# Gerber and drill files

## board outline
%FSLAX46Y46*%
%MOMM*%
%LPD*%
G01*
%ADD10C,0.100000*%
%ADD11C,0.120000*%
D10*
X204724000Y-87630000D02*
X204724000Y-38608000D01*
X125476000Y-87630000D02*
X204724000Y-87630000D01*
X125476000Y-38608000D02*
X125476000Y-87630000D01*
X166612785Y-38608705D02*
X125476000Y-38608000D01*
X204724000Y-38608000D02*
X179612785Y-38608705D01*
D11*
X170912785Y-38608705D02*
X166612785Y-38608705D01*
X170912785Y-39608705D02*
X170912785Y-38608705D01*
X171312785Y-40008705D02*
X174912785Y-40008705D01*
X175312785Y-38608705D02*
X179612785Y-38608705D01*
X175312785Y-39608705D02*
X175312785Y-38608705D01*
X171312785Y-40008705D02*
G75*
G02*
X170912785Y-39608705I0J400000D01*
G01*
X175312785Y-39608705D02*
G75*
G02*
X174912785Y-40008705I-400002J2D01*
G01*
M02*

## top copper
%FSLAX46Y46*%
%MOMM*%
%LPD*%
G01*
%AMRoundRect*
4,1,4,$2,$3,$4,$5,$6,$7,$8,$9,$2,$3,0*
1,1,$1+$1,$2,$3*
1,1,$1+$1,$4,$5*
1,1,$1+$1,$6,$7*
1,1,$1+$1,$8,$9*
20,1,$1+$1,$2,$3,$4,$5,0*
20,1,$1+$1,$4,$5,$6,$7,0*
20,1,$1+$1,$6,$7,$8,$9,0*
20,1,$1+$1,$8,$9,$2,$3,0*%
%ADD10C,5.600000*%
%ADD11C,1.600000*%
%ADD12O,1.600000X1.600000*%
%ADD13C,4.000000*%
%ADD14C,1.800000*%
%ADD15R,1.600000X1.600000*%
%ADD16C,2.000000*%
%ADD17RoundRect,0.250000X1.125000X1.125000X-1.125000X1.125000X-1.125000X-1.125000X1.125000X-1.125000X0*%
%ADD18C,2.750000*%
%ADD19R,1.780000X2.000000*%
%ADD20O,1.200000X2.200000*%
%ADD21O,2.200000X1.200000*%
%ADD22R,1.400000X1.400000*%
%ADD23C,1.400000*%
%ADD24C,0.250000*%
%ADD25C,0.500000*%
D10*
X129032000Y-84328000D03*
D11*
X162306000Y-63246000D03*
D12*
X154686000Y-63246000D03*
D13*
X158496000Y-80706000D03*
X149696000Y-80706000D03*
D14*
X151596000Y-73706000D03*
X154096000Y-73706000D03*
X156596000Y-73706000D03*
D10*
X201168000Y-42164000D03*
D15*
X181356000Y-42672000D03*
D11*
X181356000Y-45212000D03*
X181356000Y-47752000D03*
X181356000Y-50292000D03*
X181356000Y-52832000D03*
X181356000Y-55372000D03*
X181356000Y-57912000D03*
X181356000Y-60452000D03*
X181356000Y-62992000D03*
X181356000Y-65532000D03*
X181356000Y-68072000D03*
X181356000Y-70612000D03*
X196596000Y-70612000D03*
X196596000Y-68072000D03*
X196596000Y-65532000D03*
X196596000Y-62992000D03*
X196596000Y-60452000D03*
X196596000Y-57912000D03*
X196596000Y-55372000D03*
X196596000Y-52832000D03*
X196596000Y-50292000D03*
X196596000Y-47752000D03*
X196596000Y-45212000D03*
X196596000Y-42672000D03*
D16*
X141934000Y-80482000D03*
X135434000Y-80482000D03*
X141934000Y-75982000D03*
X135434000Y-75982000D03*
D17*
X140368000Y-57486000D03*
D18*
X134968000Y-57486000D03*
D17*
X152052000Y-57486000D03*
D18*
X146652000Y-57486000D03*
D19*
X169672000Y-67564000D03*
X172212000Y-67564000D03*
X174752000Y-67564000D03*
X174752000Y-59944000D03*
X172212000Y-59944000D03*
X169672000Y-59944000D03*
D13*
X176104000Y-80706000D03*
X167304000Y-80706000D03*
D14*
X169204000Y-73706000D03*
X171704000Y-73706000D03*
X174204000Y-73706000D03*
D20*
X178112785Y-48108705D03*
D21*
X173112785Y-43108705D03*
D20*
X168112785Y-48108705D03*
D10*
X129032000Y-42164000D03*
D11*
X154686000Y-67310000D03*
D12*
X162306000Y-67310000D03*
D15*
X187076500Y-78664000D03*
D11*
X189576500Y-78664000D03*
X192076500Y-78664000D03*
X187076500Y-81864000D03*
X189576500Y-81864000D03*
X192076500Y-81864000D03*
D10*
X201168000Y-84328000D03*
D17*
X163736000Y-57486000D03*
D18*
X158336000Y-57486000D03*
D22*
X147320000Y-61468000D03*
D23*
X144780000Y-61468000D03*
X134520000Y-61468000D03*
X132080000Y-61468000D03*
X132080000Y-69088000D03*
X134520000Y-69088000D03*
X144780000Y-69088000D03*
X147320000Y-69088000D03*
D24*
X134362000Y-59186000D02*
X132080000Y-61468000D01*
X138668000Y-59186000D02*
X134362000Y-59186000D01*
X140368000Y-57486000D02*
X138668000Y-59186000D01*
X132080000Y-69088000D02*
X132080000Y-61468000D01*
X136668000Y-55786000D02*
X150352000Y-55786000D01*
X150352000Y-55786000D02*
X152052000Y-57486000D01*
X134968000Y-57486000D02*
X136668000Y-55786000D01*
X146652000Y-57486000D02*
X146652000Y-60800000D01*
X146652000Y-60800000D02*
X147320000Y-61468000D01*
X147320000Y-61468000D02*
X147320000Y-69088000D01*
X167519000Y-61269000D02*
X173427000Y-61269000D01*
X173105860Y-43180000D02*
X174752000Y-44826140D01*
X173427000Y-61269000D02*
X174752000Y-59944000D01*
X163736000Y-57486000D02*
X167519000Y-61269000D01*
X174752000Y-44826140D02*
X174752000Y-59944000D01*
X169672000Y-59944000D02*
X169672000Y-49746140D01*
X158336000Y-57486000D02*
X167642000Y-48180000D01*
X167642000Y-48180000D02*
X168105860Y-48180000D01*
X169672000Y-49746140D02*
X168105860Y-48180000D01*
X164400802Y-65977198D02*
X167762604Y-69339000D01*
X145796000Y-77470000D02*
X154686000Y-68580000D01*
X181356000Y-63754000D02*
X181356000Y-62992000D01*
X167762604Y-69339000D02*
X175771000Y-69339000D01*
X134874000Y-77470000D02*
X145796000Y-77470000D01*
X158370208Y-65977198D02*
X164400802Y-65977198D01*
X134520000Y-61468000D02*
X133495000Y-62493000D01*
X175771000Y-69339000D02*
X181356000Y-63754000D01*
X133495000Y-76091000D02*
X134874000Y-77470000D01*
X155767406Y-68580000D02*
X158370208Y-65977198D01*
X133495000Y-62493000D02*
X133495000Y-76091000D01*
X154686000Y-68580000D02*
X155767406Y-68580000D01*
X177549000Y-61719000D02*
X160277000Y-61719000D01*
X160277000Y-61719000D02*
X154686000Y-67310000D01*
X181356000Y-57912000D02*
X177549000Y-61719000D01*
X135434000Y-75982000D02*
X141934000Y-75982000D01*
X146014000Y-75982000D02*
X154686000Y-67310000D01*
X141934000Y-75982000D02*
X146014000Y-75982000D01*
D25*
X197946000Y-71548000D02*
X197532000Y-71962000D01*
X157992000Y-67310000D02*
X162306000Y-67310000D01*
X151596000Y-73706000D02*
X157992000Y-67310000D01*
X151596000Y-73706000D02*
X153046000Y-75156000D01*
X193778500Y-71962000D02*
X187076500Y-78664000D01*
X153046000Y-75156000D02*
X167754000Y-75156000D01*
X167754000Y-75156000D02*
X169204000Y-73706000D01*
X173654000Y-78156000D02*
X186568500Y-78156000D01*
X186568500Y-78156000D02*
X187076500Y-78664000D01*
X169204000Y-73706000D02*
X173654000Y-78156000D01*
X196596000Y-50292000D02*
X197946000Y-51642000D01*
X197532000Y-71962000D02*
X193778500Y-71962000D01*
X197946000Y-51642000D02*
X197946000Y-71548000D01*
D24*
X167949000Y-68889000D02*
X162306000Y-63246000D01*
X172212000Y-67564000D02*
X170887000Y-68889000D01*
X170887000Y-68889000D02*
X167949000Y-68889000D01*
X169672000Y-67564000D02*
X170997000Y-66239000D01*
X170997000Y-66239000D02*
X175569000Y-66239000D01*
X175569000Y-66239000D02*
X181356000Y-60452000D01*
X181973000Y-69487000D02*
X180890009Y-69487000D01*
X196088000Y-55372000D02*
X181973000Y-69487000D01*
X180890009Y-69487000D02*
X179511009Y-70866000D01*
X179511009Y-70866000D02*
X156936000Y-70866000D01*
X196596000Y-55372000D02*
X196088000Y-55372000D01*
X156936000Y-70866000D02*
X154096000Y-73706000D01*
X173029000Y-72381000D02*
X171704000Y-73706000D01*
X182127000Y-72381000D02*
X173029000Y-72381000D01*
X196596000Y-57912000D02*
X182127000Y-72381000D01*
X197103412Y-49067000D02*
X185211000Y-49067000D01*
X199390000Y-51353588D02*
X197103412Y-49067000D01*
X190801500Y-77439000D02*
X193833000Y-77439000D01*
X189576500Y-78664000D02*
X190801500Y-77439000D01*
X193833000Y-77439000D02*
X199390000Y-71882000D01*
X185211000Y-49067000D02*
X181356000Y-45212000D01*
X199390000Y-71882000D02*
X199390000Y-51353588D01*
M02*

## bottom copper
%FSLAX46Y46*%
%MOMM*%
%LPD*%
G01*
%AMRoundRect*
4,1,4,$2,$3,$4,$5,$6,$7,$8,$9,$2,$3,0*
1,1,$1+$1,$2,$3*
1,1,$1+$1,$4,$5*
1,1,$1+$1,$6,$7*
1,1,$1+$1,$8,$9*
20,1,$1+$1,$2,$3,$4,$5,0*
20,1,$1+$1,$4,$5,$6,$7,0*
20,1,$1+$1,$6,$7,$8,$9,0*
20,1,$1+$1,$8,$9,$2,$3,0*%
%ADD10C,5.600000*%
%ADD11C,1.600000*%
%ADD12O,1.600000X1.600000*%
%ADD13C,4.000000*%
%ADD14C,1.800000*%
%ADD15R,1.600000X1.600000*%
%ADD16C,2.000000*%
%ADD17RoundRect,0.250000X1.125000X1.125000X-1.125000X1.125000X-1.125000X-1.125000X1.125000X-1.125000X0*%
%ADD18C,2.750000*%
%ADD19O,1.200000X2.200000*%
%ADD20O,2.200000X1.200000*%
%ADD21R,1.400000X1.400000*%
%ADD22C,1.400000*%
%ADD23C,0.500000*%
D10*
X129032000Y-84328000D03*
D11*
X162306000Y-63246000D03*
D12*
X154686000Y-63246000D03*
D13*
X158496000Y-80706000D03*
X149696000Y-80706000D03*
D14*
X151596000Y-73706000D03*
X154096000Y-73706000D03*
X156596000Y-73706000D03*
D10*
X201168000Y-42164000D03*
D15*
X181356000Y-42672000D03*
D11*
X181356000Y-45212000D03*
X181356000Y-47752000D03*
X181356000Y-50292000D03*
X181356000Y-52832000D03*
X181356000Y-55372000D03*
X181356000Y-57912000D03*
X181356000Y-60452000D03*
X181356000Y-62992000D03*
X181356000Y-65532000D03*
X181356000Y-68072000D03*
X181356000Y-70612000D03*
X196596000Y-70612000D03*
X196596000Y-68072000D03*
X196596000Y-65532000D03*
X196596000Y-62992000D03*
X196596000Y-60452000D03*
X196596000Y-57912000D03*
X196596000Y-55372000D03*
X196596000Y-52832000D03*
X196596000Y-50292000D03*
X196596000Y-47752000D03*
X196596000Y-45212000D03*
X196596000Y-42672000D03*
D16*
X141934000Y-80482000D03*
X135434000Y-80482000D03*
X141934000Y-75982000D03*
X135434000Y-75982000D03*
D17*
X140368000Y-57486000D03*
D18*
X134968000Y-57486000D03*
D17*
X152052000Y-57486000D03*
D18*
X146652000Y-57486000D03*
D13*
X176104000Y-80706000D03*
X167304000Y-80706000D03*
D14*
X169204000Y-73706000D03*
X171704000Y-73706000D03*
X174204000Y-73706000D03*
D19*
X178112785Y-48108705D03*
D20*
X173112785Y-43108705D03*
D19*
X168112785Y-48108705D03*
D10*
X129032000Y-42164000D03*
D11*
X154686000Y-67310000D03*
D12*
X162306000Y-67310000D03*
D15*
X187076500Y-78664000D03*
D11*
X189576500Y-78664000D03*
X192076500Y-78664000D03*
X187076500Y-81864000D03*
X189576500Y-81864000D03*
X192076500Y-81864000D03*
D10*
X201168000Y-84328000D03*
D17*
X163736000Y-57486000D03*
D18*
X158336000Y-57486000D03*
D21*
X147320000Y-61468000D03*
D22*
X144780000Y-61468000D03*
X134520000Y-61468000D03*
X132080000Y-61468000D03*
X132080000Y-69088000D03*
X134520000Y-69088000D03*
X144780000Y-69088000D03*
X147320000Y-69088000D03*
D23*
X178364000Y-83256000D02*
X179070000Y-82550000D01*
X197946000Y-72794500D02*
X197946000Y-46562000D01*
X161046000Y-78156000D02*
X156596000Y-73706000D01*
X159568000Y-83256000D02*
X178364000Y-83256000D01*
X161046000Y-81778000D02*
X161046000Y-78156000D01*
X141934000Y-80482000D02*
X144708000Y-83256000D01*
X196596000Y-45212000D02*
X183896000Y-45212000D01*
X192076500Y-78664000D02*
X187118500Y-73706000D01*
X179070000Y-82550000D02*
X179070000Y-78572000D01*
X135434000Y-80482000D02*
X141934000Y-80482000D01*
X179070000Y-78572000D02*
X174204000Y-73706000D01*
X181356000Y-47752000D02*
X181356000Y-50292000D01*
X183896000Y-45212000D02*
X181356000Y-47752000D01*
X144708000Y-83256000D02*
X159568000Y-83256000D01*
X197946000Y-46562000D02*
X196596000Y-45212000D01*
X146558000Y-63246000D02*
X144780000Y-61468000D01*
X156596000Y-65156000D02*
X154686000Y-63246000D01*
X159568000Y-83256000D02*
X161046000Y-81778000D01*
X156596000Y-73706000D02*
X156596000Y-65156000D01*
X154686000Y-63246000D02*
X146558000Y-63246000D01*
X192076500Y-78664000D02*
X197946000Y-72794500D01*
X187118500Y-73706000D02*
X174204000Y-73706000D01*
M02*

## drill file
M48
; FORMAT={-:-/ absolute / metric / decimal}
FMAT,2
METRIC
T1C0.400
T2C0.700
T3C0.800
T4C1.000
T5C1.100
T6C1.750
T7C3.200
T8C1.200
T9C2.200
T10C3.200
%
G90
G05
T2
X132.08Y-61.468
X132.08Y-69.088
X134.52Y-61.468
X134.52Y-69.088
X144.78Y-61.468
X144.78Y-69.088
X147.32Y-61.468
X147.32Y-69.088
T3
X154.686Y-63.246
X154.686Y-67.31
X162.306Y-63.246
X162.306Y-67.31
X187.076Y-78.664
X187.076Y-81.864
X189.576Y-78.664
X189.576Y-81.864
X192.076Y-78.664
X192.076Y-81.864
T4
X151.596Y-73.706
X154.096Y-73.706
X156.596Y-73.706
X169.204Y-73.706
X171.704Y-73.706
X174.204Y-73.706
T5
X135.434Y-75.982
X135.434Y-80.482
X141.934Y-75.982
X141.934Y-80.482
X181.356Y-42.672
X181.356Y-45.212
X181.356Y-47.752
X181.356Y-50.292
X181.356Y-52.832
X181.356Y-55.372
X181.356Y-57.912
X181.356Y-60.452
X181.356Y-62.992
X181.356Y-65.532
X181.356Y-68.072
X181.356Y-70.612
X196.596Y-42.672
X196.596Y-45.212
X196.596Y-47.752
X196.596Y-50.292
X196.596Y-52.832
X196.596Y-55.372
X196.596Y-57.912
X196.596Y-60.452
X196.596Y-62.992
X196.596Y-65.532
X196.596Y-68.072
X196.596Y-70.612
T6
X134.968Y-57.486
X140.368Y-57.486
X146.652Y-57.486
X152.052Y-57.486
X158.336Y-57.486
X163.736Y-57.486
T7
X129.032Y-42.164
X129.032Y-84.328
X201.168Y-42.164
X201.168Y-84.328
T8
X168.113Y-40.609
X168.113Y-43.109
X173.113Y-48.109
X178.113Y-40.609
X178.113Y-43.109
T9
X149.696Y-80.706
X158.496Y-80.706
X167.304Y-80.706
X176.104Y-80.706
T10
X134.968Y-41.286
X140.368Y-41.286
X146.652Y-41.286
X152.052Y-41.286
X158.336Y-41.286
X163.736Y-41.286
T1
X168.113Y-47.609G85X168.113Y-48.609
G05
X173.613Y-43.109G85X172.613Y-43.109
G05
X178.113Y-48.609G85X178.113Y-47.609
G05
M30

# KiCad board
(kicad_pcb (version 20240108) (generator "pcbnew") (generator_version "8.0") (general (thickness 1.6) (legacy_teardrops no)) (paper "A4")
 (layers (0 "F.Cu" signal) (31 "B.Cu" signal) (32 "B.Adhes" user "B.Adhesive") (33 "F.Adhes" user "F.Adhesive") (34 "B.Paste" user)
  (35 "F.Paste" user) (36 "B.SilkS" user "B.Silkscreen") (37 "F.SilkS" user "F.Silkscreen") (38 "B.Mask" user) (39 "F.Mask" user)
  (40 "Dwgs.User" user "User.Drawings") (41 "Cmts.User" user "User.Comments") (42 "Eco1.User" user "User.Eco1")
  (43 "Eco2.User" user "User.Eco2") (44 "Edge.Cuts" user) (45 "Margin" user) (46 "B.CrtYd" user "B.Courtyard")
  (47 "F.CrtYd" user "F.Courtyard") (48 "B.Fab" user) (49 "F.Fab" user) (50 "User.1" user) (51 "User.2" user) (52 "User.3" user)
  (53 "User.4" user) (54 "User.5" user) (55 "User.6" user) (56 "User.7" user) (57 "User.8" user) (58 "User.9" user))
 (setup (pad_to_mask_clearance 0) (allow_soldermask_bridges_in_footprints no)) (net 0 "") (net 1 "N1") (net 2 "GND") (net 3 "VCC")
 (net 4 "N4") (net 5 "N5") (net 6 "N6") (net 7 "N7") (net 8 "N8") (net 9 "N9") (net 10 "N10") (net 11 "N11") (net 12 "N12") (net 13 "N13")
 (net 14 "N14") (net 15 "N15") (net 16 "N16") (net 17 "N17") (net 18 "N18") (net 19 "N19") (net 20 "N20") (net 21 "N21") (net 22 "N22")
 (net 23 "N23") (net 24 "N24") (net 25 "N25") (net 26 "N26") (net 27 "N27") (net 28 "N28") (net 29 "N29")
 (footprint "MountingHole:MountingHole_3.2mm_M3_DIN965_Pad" (layer "F.Cu") (at 129.032 84.328)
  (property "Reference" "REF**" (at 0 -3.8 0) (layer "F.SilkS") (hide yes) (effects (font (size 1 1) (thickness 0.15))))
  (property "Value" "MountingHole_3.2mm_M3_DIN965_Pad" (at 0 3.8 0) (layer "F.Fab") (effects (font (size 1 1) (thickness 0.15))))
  (pad "1" thru_hole circle (at 0 0) (size 5.6 5.6) (drill 3.2) (layers "*.Cu" "*.Mask") (remove_unused_layers no)))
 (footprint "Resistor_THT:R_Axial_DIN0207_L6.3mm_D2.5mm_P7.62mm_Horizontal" (layer "F.Cu") (at 162.306 63.246 180)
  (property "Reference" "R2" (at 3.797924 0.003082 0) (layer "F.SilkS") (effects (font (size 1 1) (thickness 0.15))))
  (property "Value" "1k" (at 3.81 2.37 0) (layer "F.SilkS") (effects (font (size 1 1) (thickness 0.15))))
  (pad "1" thru_hole circle (at 0 0 180) (size 1.6 1.6) (drill 0.8) (layers "*.Cu" "*.Mask") (remove_unused_layers no) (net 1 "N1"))
  (pad "2" thru_hole oval (at 7.62 0 180) (size 1.6 1.6) (drill 0.8) (layers "*.Cu" "*.Mask") (remove_unused_layers no) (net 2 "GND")))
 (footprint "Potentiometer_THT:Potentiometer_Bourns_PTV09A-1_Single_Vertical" (layer "F.Cu") (at 151.596 73.706 -90)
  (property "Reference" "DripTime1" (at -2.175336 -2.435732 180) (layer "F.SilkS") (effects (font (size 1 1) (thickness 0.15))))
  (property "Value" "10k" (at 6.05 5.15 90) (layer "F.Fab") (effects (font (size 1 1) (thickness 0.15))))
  (pad "" np_thru_hole circle (at 7 -6.9 270) (size 4 4) (drill 2.2) (layers "F&B.Cu" "*.Mask"))
  (pad "" np_thru_hole circle (at 7 1.9 270) (size 4 4) (drill 2.2) (layers "F&B.Cu" "*.Mask"))
  (pad "1" thru_hole circle (at 0 0 270) (size 1.8 1.8) (drill 1) (layers "*.Cu" "*.Mask") (remove_unused_layers no) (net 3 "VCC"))
  (pad "2" thru_hole circle (at 0 -2.5 270) (size 1.8 1.8) (drill 1) (layers "*.Cu" "*.Mask") (remove_unused_layers no) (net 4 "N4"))
  (pad "3" thru_hole circle (at 0 -5 270) (size 1.8 1.8) (drill 1) (layers "*.Cu" "*.Mask") (remove_unused_layers no) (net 2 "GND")))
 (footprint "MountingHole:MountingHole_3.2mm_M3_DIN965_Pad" (layer "F.Cu") (at 201.168 42.164)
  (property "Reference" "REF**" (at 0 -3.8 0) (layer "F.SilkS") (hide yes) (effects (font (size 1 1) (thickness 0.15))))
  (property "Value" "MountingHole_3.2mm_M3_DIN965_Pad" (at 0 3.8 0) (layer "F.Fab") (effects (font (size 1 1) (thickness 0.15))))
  (pad "1" thru_hole circle (at 0 0) (size 5.6 5.6) (drill 3.2) (layers "*.Cu" "*.Mask") (remove_unused_layers no)))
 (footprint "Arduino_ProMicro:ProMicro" (layer "F.Cu") (at 188.976 56.642 -90)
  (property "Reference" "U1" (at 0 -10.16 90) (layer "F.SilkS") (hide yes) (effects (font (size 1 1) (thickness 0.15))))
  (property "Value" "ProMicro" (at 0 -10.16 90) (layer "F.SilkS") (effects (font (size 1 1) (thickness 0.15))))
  (pad "1" thru_hole rect (at -13.97 7.62 270) (size 1.6 1.6) (drill 1.1) (layers "*.Cu" "*.Mask" "F.SilkS") (remove_unused_layers no)
   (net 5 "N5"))
  (pad "2" thru_hole circle (at -11.43 7.62 270) (size 1.6 1.6) (drill 1.1) (layers "*.Cu" "*.Mask" "F.SilkS") (remove_unused_layers no)
   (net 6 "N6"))
  (pad "3" thru_hole circle (at -8.89 7.62 270) (size 1.6 1.6) (drill 1.1) (layers "*.Cu" "*.Mask" "F.SilkS") (remove_unused_layers no)
   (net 2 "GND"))
  (pad "4" thru_hole circle (at -6.35 7.62 270) (size 1.6 1.6) (drill 1.1) (layers "*.Cu" "*.Mask" "F.SilkS") (remove_unused_layers no)
   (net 2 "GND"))
  (pad "5" thru_hole circle (at -3.81 7.62 270) (size 1.6 1.6) (drill 1.1) (layers "*.Cu" "*.Mask" "F.SilkS") (remove_unused_layers no)
   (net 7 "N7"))
  (pad "6" thru_hole circle (at -1.27 7.62 270) (size 1.6 1.6) (drill 1.1) (layers "*.Cu" "*.Mask" "F.SilkS") (remove_unused_layers no)
   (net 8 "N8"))
  (pad "7" thru_hole circle (at 1.27 7.62 270) (size 1.6 1.6) (drill 1.1) (layers "*.Cu" "*.Mask" "F.SilkS") (remove_unused_layers no)
   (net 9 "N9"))
  (pad "8" thru_hole circle (at 3.81 7.62 270) (size 1.6 1.6) (drill 1.1) (layers "*.Cu" "*.Mask" "F.SilkS") (remove_unused_layers no)
   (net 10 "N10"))
  (pad "9" thru_hole circle (at 6.35 7.62 270) (size 1.6 1.6) (drill 1.1) (layers "*.Cu" "*.Mask" "F.SilkS") (remove_unused_layers no)
   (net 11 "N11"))
  (pad "10" thru_hole circle (at 8.89 7.62 270) (size 1.6 1.6) (drill 1.1) (layers "*.Cu" "*.Mask" "F.SilkS") (remove_unused_layers no)
   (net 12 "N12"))
  (pad "11" thru_hole circle (at 11.43 7.62 270) (size 1.6 1.6) (drill 1.1) (layers "*.Cu" "*.Mask" "F.SilkS") (remove_unused_layers no)
   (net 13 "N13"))
  (pad "12" thru_hole circle (at 13.97 7.62 270) (size 1.6 1.6) (drill 1.1) (layers "*.Cu" "*.Mask" "F.SilkS") (remove_unused_layers no)
   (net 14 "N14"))
  (pad "13" thru_hole circle (at 13.97 -7.62 270) (size 1.6 1.6) (drill 1.1) (layers "*.Cu" "*.Mask" "F.SilkS") (remove_unused_layers no)
   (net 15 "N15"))
  (pad "14" thru_hole circle (at 11.43 -7.62 270) (size 1.6 1.6) (drill 1.1) (layers "*.Cu" "*.Mask" "F.SilkS") (remove_unused_layers no)
   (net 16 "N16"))
  (pad "15" thru_hole circle (at 8.89 -7.62 270) (size 1.6 1.6) (drill 1.1) (layers "*.Cu" "*.Mask" "F.SilkS") (remove_unused_layers no)
   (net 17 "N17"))
  (pad "16" thru_hole circle (at 6.35 -7.62 270) (size 1.6 1.6) (drill 1.1) (layers "*.Cu" "*.Mask" "F.SilkS") (remove_unused_layers no)
   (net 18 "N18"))
  (pad "17" thru_hole circle (at 3.81 -7.62 270) (size 1.6 1.6) (drill 1.1) (layers "*.Cu" "*.Mask" "F.SilkS") (remove_unused_layers no)
   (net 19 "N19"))
  (pad "18" thru_hole circle (at 1.27 -7.62 270) (size 1.6 1.6) (drill 1.1) (layers "*.Cu" "*.Mask" "F.SilkS") (remove_unused_layers no)
   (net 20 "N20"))
  (pad "19" thru_hole circle (at -1.27 -7.62 270) (size 1.6 1.6) (drill 1.1) (layers "*.Cu" "*.Mask" "F.SilkS") (remove_unused_layers no)
   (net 4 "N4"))
  (pad "20" thru_hole circle (at -3.81 -7.62 270) (size 1.6 1.6) (drill 1.1) (layers "*.Cu" "*.Mask" "F.SilkS") (remove_unused_layers no)
   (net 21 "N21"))
  (pad "21" thru_hole circle (at -6.35 -7.62 270) (size 1.6 1.6) (drill 1.1) (layers "*.Cu" "*.Mask" "F.SilkS") (remove_unused_layers no)
   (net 3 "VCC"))
  (pad "22" thru_hole circle (at -8.89 -7.62 270) (size 1.6 1.6) (drill 1.1) (layers "*.Cu" "*.Mask" "F.SilkS") (remove_unused_layers no)
   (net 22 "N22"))
  (pad "23" thru_hole circle (at -11.43 -7.62 270) (size 1.6 1.6) (drill 1.1) (layers "*.Cu" "*.Mask" "F.SilkS") (remove_unused_layers no)
   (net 2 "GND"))
  (pad "24" thru_hole circle (at -13.97 -7.62 270) (size 1.6 1.6) (drill 1.1) (layers "*.Cu" "*.Mask" "F.SilkS") (remove_unused_layers no)
   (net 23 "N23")))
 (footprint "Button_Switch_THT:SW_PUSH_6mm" (layer "F.Cu") (at 141.934 80.482 180)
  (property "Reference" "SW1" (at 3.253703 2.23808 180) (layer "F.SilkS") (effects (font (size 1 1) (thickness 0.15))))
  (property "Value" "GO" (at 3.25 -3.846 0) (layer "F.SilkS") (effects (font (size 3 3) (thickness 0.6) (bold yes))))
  (pad "1" thru_hole circle (at 0 0 270) (size 2 2) (drill 1.1) (layers "*.Cu" "*.Mask") (remove_unused_layers no) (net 2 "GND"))
  (pad "1" thru_hole circle (at 6.5 0 270) (size 2 2) (drill 1.1) (layers "*.Cu" "*.Mask") (remove_unused_layers no) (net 2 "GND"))
  (pad "2" thru_hole circle (at 0 4.5 270) (size 2 2) (drill 1.1) (layers "*.Cu" "*.Mask") (remove_unused_layers no) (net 9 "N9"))
  (pad "2" thru_hole circle (at 6.5 4.5 270) (size 2 2) (drill 1.1) (layers "*.Cu" "*.Mask") (remove_unused_layers no) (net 9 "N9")))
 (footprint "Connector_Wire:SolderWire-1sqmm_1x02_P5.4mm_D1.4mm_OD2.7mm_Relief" (layer "F.Cu") (at 140.368 57.486 180)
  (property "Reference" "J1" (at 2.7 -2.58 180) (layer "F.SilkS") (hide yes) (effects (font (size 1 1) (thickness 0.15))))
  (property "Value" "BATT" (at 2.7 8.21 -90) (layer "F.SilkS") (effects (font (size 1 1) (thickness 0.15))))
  (pad "" np_thru_hole circle (at 0 16.2 180) (size 3.2 3.2) (drill 3.2) (layers "*.Cu" "*.Mask"))
  (pad "" np_thru_hole circle (at 5.4 16.2 180) (size 3.2 3.2) (drill 3.2) (layers "*.Cu" "*.Mask"))
  (pad "1" thru_hole roundrect (at 0 0 180) (size 2.75 2.75) (drill 1.75) (layers "*.Cu" "*.Mask") (remove_unused_layers no)
   (roundrect_rratio 0.090909) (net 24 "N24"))
  (pad "2" thru_hole circle (at 5.4 0 180) (size 2.75 2.75) (drill 1.75) (layers "*.Cu" "*.Mask") (remove_unused_layers no) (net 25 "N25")))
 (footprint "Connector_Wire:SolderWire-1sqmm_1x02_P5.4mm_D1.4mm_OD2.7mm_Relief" (layer "F.Cu") (at 152.052 57.486 180)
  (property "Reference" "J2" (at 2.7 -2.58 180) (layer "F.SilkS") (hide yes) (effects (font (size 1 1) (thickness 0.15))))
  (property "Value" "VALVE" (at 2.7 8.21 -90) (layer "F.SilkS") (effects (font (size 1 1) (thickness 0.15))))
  (pad "" np_thru_hole circle (at 0 16.2 180) (size 3.2 3.2) (drill 3.2) (layers "*.Cu" "*.Mask"))
  (pad "" np_thru_hole circle (at 5.4 16.2 180) (size 3.2 3.2) (drill 3.2) (layers "*.Cu" "*.Mask"))
  (pad "1" thru_hole roundrect (at 0 0 180) (size 2.75 2.75) (drill 1.75) (layers "*.Cu" "*.Mask") (remove_unused_layers no)
   (roundrect_rratio 0.090909) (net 25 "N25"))
  (pad "2" thru_hole circle (at 5.4 0 180) (size 2.75 2.75) (drill 1.75) (layers "*.Cu" "*.Mask") (remove_unused_layers no) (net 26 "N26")))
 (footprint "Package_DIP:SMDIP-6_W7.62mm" (layer "F.Cu") (at 172.212 63.754 90)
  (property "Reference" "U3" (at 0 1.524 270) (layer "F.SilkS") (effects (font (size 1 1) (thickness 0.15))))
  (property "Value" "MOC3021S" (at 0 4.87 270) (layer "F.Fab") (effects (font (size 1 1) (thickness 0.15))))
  (pad "1" smd rect (at -3.81 -2.54 90) (size 2 1.78) (layers "F.Cu" "F.Paste" "F.Mask") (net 10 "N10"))
  (pad "2" smd rect (at -3.81 0 90) (size 2 1.78) (layers "F.Cu" "F.Paste" "F.Mask") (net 1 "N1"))
  (pad "3" smd rect (at -3.81 2.54 90) (size 2 1.78) (layers "F.Cu" "F.Paste" "F.Mask") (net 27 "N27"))
  (pad "4" smd rect (at 3.81 2.54 90) (size 2 1.78) (layers "F.Cu" "F.Paste" "F.Mask") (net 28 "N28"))
  (pad "5" smd rect (at 3.81 0 90) (size 2 1.78) (layers "F.Cu" "F.Paste" "F.Mask"))
  (pad "6" smd rect (at 3.81 -2.54 90) (size 2 1.78) (layers "F.Cu" "F.Paste" "F.Mask") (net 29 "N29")))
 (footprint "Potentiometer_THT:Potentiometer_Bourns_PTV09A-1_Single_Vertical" (layer "F.Cu") (at 169.204 73.706 -90)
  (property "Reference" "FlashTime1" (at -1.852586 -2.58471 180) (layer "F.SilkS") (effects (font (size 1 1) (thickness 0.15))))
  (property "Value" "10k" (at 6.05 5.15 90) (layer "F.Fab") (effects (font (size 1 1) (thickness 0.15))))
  (pad "" np_thru_hole circle (at 7 -6.9 270) (size 4 4) (drill 2.2) (layers "F&B.Cu" "*.Mask"))
  (pad "" np_thru_hole circle (at 7 1.9 270) (size 4 4) (drill 2.2) (layers "F&B.Cu" "*.Mask"))
  (pad "1" thru_hole circle (at 0 0 270) (size 1.8 1.8) (drill 1) (layers "*.Cu" "*.Mask") (remove_unused_layers no) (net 3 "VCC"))
  (pad "2" thru_hole circle (at 0 -2.5 270) (size 1.8 1.8) (drill 1) (layers "*.Cu" "*.Mask") (remove_unused_layers no) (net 20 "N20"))
  (pad "3" thru_hole circle (at 0 -5 270) (size 1.8 1.8) (drill 1) (layers "*.Cu" "*.Mask") (remove_unused_layers no) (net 2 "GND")))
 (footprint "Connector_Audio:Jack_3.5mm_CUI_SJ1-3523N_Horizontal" (layer "F.Cu") (at 173.112785 43.108705 180)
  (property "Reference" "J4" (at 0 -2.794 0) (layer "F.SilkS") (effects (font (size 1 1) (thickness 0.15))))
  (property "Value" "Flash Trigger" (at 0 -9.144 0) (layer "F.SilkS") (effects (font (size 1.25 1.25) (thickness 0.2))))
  (fp_line (start 2.2 4.5) (end 6.5 4.5) (stroke (width 0.12) (type solid)) (layer "Edge.Cuts"))
  (fp_line (start 2.2 3.5) (end 2.2 4.5) (stroke (width 0.12) (type solid)) (layer "Edge.Cuts"))
  (fp_line (start 1.8 3.1) (end -1.8 3.1) (stroke (width 0.12) (type solid)) (layer "Edge.Cuts"))
  (fp_line (start -2.2 4.5) (end -6.5 4.5) (stroke (width 0.12) (type solid)) (layer "Edge.Cuts"))
  (fp_line (start -2.2 3.5) (end -2.2 4.5) (stroke (width 0.12) (type solid)) (layer "Edge.Cuts"))
  (fp_arc (start 1.8 3.1) (mid 2.082843 3.217157) (end 2.2 3.5) (stroke (width 0.12) (type solid)) (layer "Edge.Cuts"))
  (fp_arc (start -2.2 3.5) (mid -2.082842 3.217158) (end -1.8 3.1) (stroke (width 0.12) (type solid)) (layer "Edge.Cuts"))
  (pad "" np_thru_hole circle (at -5 0 180) (size 1.2 1.2) (drill 1.2) (layers "*.Cu"))
  (pad "" np_thru_hole circle (at -5 2.5 180) (size 1.2 1.2) (drill 1.2) (layers "*.Cu"))
  (pad "" np_thru_hole circle (at 0 -5 180) (size 1.2 1.2) (drill 1.2) (layers "*.Cu"))
  (pad "" np_thru_hole circle (at 5 0 180) (size 1.2 1.2) (drill 1.2) (layers "*.Cu"))
  (pad "" np_thru_hole circle (at 5 2.5 180) (size 1.2 1.2) (drill 1.2) (layers "*.Cu"))
  (pad "R" thru_hole oval (at -5 -5 180) (size 1.2 2.2) (drill oval 0.4 1.4) (layers "*.Cu" "*.Mask") (remove_unused_layers no))
  (pad "S" thru_hole oval (at 0 0 180) (size 2.2 1.2) (drill oval 1.4 0.4) (layers "*.Cu" "*.Mask") (remove_unused_layers no) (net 28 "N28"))
  (pad "T" thru_hole oval (at 5 -5) (size 1.2 2.2) (drill oval 0.4 1.4) (layers "*.Cu" "*.Mask") (remove_unused_layers no) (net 29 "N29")))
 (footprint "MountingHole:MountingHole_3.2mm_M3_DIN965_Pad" (layer "F.Cu") (at 129.032 42.164)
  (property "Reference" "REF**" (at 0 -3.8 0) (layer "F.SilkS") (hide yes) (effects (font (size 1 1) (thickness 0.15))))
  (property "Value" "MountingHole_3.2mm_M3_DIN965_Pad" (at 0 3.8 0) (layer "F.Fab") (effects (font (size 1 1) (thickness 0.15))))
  (pad "1" thru_hole circle (at 0 0) (size 5.6 5.6) (drill 3.2) (layers "*.Cu" "*.Mask") (remove_unused_layers no)))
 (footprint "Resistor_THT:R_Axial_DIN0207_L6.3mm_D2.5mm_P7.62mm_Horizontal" (layer "F.Cu") (at 154.686 67.31)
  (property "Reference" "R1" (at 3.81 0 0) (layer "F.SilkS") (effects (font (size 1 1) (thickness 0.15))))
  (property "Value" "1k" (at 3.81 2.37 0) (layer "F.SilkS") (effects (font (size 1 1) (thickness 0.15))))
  (pad "1" thru_hole circle (at 0 0) (size 1.6 1.6) (drill 0.8) (layers "*.Cu" "*.Mask") (remove_unused_layers no) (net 9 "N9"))
  (pad "2" thru_hole oval (at 7.62 0) (size 1.6 1.6) (drill 0.8) (layers "*.Cu" "*.Mask") (remove_unused_layers no) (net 3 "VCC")))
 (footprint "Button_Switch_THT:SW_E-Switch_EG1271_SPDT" (layer "F.Cu") (at 187.0765 78.664)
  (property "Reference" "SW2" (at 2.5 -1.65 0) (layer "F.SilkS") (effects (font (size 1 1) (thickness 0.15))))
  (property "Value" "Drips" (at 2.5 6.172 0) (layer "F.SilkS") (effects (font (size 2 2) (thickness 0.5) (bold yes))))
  (pad "1" thru_hole rect (at 0 0) (size 1.6 1.6) (drill 0.8) (layers "*.Cu" "*.Mask") (remove_unused_layers no) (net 3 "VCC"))
  (pad "2" thru_hole circle (at 2.5 0) (size 1.6 1.6) (drill 0.8) (layers "*.Cu" "*.Mask") (remove_unused_layers no) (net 6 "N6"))
  (pad "3" thru_hole circle (at 5 0) (size 1.6 1.6) (drill 0.8) (layers "*.Cu" "*.Mask") (remove_unused_layers no) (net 2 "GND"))
  (pad "4" thru_hole circle (at 0 3.2) (size 1.6 1.6) (drill 0.8) (layers "*.Cu" "*.Mask") (remove_unused_layers no))
  (pad "5" thru_hole circle (at 2.5 3.2) (size 1.6 1.6) (drill 0.8) (layers "*.Cu" "*.Mask") (remove_unused_layers no))
  (pad "6" thru_hole circle (at 5 3.2) (size 1.6 1.6) (drill 0.8) (layers "*.Cu" "*.Mask") (remove_unused_layers no)))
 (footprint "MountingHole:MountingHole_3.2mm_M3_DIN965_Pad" (layer "F.Cu") (at 201.168 84.328)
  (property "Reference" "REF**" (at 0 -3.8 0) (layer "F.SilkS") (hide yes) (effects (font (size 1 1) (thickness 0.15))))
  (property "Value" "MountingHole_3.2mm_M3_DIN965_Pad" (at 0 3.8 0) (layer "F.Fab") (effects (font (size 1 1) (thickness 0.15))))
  (pad "1" thru_hole circle (at 0 0) (size 5.6 5.6) (drill 3.2) (layers "*.Cu" "*.Mask") (remove_unused_layers no)))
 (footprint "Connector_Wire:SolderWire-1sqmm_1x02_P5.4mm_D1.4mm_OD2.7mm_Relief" (layer "F.Cu") (at 163.736 57.486 180)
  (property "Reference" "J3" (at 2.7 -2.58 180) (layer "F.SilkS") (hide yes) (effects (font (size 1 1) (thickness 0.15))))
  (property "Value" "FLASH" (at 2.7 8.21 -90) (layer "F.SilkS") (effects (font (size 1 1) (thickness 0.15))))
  (pad "" np_thru_hole circle (at 0 16.2 180) (size 3.2 3.2) (drill 3.2) (layers "*.Cu" "*.Mask"))
  (pad "" np_thru_hole circle (at 5.4 16.2 180) (size 3.2 3.2) (drill 3.2) (layers "*.Cu" "*.Mask"))
  (pad "1" thru_hole roundrect (at 0 0 180) (size 2.75 2.75) (drill 1.75) (layers "*.Cu" "*.Mask") (remove_unused_layers no)
   (roundrect_rratio 0.090909) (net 28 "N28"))
  (pad "2" thru_hole circle (at 5.4 0 180) (size 2.75 2.75) (drill 1.75) (layers "*.Cu" "*.Mask") (remove_unused_layers no) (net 29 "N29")))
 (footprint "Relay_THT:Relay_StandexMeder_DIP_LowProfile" (layer "F.Cu") (at 147.32 61.468 -90)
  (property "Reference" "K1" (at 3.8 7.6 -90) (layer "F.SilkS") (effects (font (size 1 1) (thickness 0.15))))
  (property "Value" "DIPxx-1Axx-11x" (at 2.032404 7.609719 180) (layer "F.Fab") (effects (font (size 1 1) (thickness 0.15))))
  (pad "1" thru_hole rect (at 0 0 270) (size 1.4 1.4) (drill 0.7) (layers "*.Cu" "*.Mask") (remove_unused_layers no) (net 26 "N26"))
  (pad "2" thru_hole circle (at 0 2.54 270) (size 1.4 1.4) (drill 0.7) (layers "*.Cu" "*.Mask") (remove_unused_layers no) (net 2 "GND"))
  (pad "6" thru_hole circle (at 0 12.8 270) (size 1.4 1.4) (drill 0.7) (layers "*.Cu" "*.Mask") (remove_unused_layers no) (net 11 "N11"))
  (pad "7" thru_hole circle (at 0 15.24 270) (size 1.4 1.4) (drill 0.7) (layers "*.Cu" "*.Mask") (remove_unused_layers no) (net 24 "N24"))
  (pad "8" thru_hole circle (at 7.62 15.24 270) (size 1.4 1.4) (drill 0.7) (layers "*.Cu" "*.Mask") (remove_unused_layers no) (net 24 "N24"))
  (pad "9" thru_hole circle (at 7.62 12.8 270) (size 1.4 1.4) (drill 0.7) (layers "*.Cu" "*.Mask") (remove_unused_layers no))
  (pad "13" thru_hole circle (at 7.62 2.54 270) (size 1.4 1.4) (drill 0.7) (layers "*.Cu" "*.Mask") (remove_unused_layers no))
  (pad "14" thru_hole circle (at 7.62 0 270) (size 1.4 1.4) (drill 0.7) (layers "*.Cu" "*.Mask") (remove_unused_layers no) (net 26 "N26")))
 (gr_line (start 204.724 87.63) (end 204.724 38.608) (stroke (width 0.1) (type default)) (layer "Edge.Cuts"))
 (gr_line (start 125.476 87.63) (end 204.724 87.63) (stroke (width 0.1) (type default)) (layer "Edge.Cuts"))
 (gr_line (start 125.476 38.608) (end 125.476 87.63) (stroke (width 0.1) (type default)) (layer "Edge.Cuts"))
 (gr_line (start 166.612785 38.608705) (end 125.476 38.608) (stroke (width 0.1) (type default)) (layer "Edge.Cuts"))
 (gr_line (start 204.724 38.608) (end 179.612785 38.608705) (stroke (width 0.1) (type default)) (layer "Edge.Cuts"))
 (segment (start 134.362 59.186) (end 132.08 61.468) (width 0.25) (layer "F.Cu") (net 24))
 (segment (start 138.668 59.186) (end 134.362 59.186) (width 0.25) (layer "F.Cu") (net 24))
 (segment (start 140.368 57.486) (end 138.668 59.186) (width 0.25) (layer "F.Cu") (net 24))
 (segment (start 132.08 69.088) (end 132.08 61.468) (width 0.25) (layer "F.Cu") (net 24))
 (segment (start 136.668 55.786) (end 150.352 55.786) (width 0.25) (layer "F.Cu") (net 25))
 (segment (start 150.352 55.786) (end 152.052 57.486) (width 0.25) (layer "F.Cu") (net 25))
 (segment (start 134.968 57.486) (end 136.668 55.786) (width 0.25) (layer "F.Cu") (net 25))
 (segment (start 146.652 57.486) (end 146.652 60.8) (width 0.25) (layer "F.Cu") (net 26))
 (segment (start 146.652 60.8) (end 147.32 61.468) (width 0.25) (layer "F.Cu") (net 26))
 (segment (start 147.32 61.468) (end 147.32 69.088) (width 0.25) (layer "F.Cu") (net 26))
 (segment (start 167.519 61.269) (end 173.427 61.269) (width 0.25) (layer "F.Cu") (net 28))
 (segment (start 173.10586 43.18) (end 174.752 44.82614) (width 0.25) (layer "F.Cu") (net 28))
 (segment (start 173.427 61.269) (end 174.752 59.944) (width 0.25) (layer "F.Cu") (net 28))
 (segment (start 163.736 57.486) (end 167.519 61.269) (width 0.25) (layer "F.Cu") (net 28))
 (segment (start 174.752 44.82614) (end 174.752 59.944) (width 0.25) (layer "F.Cu") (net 28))
 (segment (start 169.672 59.944) (end 169.672 49.74614) (width 0.25) (layer "F.Cu") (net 29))
 (segment (start 158.336 57.486) (end 167.642 48.18) (width 0.25) (layer "F.Cu") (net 29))
 (segment (start 167.642 48.18) (end 168.10586 48.18) (width 0.25) (layer "F.Cu") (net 29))
 (segment (start 169.672 49.74614) (end 168.10586 48.18) (width 0.25) (layer "F.Cu") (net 29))
 (segment (start 164.400802 65.977198) (end 167.762604 69.339) (width 0.25) (layer "F.Cu") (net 11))
 (segment (start 145.796 77.47) (end 154.686 68.58) (width 0.25) (layer "F.Cu") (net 11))
 (segment (start 181.356 63.754) (end 181.356 62.992) (width 0.25) (layer "F.Cu") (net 11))
 (segment (start 167.762604 69.339) (end 175.771 69.339) (width 0.25) (layer "F.Cu") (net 11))
 (segment (start 134.874 77.47) (end 145.796 77.47) (width 0.25) (layer "F.Cu") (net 11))
 (segment (start 158.370208 65.977198) (end 164.400802 65.977198) (width 0.25) (layer "F.Cu") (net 11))
 (segment (start 134.52 61.468) (end 133.495 62.493) (width 0.25) (layer "F.Cu") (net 11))
 (segment (start 175.771 69.339) (end 181.356 63.754) (width 0.25) (layer "F.Cu") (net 11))
 (segment (start 133.495 76.091) (end 134.874 77.47) (width 0.25) (layer "F.Cu") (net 11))
 (segment (start 155.767406 68.58) (end 158.370208 65.977198) (width 0.25) (layer "F.Cu") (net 11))
 (segment (start 133.495 62.493) (end 133.495 76.091) (width 0.25) (layer "F.Cu") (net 11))
 (segment (start 154.686 68.58) (end 155.767406 68.58) (width 0.25) (layer "F.Cu") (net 11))
 (segment (start 177.549 61.719) (end 160.277 61.719) (width 0.25) (layer "F.Cu") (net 9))
 (segment (start 160.277 61.719) (end 154.686 67.31) (width 0.25) (layer "F.Cu") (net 9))
 (segment (start 181.356 57.912) (end 177.549 61.719) (width 0.25) (layer "F.Cu") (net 9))
 (segment (start 135.434 75.982) (end 141.934 75.982) (width 0.25) (layer "F.Cu") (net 9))
 (segment (start 146.014 75.982) (end 154.686 67.31) (width 0.25) (layer "F.Cu") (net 9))
 (segment (start 141.934 75.982) (end 146.014 75.982) (width 0.25) (layer "F.Cu") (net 9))
 (segment (start 197.946 71.548) (end 197.532 71.962) (width 0.5) (layer "F.Cu") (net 3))
 (segment (start 157.992 67.31) (end 162.306 67.31) (width 0.5) (layer "F.Cu") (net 3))
 (segment (start 151.596 73.706) (end 157.992 67.31) (width 0.5) (layer "F.Cu") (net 3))
 (segment (start 151.596 73.706) (end 153.046 75.156) (width 0.5) (layer "F.Cu") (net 3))
 (segment (start 193.7785 71.962) (end 187.0765 78.664) (width 0.5) (layer "F.Cu") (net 3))
 (segment (start 153.046 75.156) (end 167.754 75.156) (width 0.5) (layer "F.Cu") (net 3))
 (segment (start 167.754 75.156) (end 169.204 73.706) (width 0.5) (layer "F.Cu") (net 3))
 (segment (start 173.654 78.156) (end 186.5685 78.156) (width 0.5) (layer "F.Cu") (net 3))
 (segment (start 186.5685 78.156) (end 187.0765 78.664) (width 0.5) (layer "F.Cu") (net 3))
 (segment (start 169.204 73.706) (end 173.654 78.156) (width 0.5) (layer "F.Cu") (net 3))
 (segment (start 196.596 50.292) (end 197.946 51.642) (width 0.5) (layer "F.Cu") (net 3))
 (segment (start 197.532 71.962) (end 193.7785 71.962) (width 0.5) (layer "F.Cu") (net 3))
 (segment (start 197.946 51.642) (end 197.946 71.548) (width 0.5) (layer "F.Cu") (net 3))
 (segment (start 167.949 68.889) (end 162.306 63.246) (width 0.25) (layer "F.Cu") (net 1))
 (segment (start 172.212 67.564) (end 170.887 68.889) (width 0.25) (layer "F.Cu") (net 1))
 (segment (start 170.887 68.889) (end 167.949 68.889) (width 0.25) (layer "F.Cu") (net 1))
 (segment (start 178.364 83.256) (end 179.07 82.55) (width 0.5) (layer "B.Cu") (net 2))
 (segment (start 197.946 72.7945) (end 197.946 46.562) (width 0.5) (layer "B.Cu") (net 2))
 (segment (start 161.046 78.156) (end 156.596 73.706) (width 0.5) (layer "B.Cu") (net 2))
 (segment (start 159.568 83.256) (end 178.364 83.256) (width 0.5) (layer "B.Cu") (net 2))
 (segment (start 161.046 81.778) (end 161.046 78.156) (width 0.5) (layer "B.Cu") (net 2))
 (segment (start 141.934 80.482) (end 144.708 83.256) (width 0.5) (layer "B.Cu") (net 2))
 (segment (start 196.596 45.212) (end 183.896 45.212) (width 0.5) (layer "B.Cu") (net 2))
 (segment (start 192.0765 78.664) (end 187.1185 73.706) (width 0.5) (layer "B.Cu") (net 2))
 (segment (start 179.07 82.55) (end 179.07 78.572) (width 0.5) (layer "B.Cu") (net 2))
 (segment (start 135.434 80.482) (end 141.934 80.482) (width 0.5) (layer "B.Cu") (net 2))
 (segment (start 179.07 78.572) (end 174.204 73.706) (width 0.5) (layer "B.Cu") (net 2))
 (segment (start 181.356 47.752) (end 181.356 50.292) (width 0.5) (layer "B.Cu") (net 2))
 (segment (start 183.896 45.212) (end 181.356 47.752) (width 0.5) (layer "B.Cu") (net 2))
 (segment (start 144.708 83.256) (end 159.568 83.256) (width 0.5) (layer "B.Cu") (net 2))
 (segment (start 197.946 46.562) (end 196.596 45.212) (width 0.5) (layer "B.Cu") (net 2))
 (segment (start 146.558 63.246) (end 144.78 61.468) (width 0.5) (layer "B.Cu") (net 2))
 (segment (start 156.596 65.156) (end 154.686 63.246) (width 0.5) (layer "B.Cu") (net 2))
 (segment (start 159.568 83.256) (end 161.046 81.778) (width 0.5) (layer "B.Cu") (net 2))
 (segment (start 156.596 73.706) (end 156.596 65.156) (width 0.5) (layer "B.Cu") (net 2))
 (segment (start 154.686 63.246) (end 146.558 63.246) (width 0.5) (layer "B.Cu") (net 2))
 (segment (start 192.0765 78.664) (end 197.946 72.7945) (width 0.5) (layer "B.Cu") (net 2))
 (segment (start 187.1185 73.706) (end 174.204 73.706) (width 0.5) (layer "B.Cu") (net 2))
 (segment (start 169.672 67.564) (end 170.997 66.239) (width 0.25) (layer "F.Cu") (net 10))
 (segment (start 170.997 66.239) (end 175.569 66.239) (width 0.25) (layer "F.Cu") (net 10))
 (segment (start 175.569 66.239) (end 181.356 60.452) (width 0.25) (layer "F.Cu") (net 10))
 (segment (start 181.973 69.487) (end 180.890009 69.487) (width 0.25) (layer "F.Cu") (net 4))
 (segment (start 196.088 55.372) (end 181.973 69.487) (width 0.25) (layer "F.Cu") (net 4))
 (segment (start 180.890009 69.487) (end 179.511009 70.866) (width 0.25) (layer "F.Cu") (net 4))
 (segment (start 179.511009 70.866) (end 156.936 70.866) (width 0.25) (layer "F.Cu") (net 4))
 (segment (start 196.596 55.372) (end 196.088 55.372) (width 0.25) (layer "F.Cu") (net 4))
 (segment (start 156.936 70.866) (end 154.096 73.706) (width 0.25) (layer "F.Cu") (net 4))
 (segment (start 173.029 72.381) (end 171.704 73.706) (width 0.25) (layer "F.Cu") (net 20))
 (segment (start 182.127 72.381) (end 173.029 72.381) (width 0.25) (layer "F.Cu") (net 20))
 (segment (start 196.596 57.912) (end 182.127 72.381) (width 0.25) (layer "F.Cu") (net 20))
 (segment (start 197.103412 49.067) (end 185.211 49.067) (width 0.25) (layer "F.Cu") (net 6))
 (segment (start 199.39 51.353588) (end 197.103412 49.067) (width 0.25) (layer "F.Cu") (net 6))
 (segment (start 190.8015 77.439) (end 193.833 77.439) (width 0.25) (layer "F.Cu") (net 6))
 (segment (start 189.5765 78.664) (end 190.8015 77.439) (width 0.25) (layer "F.Cu") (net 6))
 (segment (start 193.833 77.439) (end 199.39 71.882) (width 0.25) (layer "F.Cu") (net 6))
 (segment (start 185.211 49.067) (end 181.356 45.212) (width 0.25) (layer "F.Cu") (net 6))
 (segment (start 199.39 71.882) (end 199.39 51.353588) (width 0.25) (layer "F.Cu") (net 6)))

